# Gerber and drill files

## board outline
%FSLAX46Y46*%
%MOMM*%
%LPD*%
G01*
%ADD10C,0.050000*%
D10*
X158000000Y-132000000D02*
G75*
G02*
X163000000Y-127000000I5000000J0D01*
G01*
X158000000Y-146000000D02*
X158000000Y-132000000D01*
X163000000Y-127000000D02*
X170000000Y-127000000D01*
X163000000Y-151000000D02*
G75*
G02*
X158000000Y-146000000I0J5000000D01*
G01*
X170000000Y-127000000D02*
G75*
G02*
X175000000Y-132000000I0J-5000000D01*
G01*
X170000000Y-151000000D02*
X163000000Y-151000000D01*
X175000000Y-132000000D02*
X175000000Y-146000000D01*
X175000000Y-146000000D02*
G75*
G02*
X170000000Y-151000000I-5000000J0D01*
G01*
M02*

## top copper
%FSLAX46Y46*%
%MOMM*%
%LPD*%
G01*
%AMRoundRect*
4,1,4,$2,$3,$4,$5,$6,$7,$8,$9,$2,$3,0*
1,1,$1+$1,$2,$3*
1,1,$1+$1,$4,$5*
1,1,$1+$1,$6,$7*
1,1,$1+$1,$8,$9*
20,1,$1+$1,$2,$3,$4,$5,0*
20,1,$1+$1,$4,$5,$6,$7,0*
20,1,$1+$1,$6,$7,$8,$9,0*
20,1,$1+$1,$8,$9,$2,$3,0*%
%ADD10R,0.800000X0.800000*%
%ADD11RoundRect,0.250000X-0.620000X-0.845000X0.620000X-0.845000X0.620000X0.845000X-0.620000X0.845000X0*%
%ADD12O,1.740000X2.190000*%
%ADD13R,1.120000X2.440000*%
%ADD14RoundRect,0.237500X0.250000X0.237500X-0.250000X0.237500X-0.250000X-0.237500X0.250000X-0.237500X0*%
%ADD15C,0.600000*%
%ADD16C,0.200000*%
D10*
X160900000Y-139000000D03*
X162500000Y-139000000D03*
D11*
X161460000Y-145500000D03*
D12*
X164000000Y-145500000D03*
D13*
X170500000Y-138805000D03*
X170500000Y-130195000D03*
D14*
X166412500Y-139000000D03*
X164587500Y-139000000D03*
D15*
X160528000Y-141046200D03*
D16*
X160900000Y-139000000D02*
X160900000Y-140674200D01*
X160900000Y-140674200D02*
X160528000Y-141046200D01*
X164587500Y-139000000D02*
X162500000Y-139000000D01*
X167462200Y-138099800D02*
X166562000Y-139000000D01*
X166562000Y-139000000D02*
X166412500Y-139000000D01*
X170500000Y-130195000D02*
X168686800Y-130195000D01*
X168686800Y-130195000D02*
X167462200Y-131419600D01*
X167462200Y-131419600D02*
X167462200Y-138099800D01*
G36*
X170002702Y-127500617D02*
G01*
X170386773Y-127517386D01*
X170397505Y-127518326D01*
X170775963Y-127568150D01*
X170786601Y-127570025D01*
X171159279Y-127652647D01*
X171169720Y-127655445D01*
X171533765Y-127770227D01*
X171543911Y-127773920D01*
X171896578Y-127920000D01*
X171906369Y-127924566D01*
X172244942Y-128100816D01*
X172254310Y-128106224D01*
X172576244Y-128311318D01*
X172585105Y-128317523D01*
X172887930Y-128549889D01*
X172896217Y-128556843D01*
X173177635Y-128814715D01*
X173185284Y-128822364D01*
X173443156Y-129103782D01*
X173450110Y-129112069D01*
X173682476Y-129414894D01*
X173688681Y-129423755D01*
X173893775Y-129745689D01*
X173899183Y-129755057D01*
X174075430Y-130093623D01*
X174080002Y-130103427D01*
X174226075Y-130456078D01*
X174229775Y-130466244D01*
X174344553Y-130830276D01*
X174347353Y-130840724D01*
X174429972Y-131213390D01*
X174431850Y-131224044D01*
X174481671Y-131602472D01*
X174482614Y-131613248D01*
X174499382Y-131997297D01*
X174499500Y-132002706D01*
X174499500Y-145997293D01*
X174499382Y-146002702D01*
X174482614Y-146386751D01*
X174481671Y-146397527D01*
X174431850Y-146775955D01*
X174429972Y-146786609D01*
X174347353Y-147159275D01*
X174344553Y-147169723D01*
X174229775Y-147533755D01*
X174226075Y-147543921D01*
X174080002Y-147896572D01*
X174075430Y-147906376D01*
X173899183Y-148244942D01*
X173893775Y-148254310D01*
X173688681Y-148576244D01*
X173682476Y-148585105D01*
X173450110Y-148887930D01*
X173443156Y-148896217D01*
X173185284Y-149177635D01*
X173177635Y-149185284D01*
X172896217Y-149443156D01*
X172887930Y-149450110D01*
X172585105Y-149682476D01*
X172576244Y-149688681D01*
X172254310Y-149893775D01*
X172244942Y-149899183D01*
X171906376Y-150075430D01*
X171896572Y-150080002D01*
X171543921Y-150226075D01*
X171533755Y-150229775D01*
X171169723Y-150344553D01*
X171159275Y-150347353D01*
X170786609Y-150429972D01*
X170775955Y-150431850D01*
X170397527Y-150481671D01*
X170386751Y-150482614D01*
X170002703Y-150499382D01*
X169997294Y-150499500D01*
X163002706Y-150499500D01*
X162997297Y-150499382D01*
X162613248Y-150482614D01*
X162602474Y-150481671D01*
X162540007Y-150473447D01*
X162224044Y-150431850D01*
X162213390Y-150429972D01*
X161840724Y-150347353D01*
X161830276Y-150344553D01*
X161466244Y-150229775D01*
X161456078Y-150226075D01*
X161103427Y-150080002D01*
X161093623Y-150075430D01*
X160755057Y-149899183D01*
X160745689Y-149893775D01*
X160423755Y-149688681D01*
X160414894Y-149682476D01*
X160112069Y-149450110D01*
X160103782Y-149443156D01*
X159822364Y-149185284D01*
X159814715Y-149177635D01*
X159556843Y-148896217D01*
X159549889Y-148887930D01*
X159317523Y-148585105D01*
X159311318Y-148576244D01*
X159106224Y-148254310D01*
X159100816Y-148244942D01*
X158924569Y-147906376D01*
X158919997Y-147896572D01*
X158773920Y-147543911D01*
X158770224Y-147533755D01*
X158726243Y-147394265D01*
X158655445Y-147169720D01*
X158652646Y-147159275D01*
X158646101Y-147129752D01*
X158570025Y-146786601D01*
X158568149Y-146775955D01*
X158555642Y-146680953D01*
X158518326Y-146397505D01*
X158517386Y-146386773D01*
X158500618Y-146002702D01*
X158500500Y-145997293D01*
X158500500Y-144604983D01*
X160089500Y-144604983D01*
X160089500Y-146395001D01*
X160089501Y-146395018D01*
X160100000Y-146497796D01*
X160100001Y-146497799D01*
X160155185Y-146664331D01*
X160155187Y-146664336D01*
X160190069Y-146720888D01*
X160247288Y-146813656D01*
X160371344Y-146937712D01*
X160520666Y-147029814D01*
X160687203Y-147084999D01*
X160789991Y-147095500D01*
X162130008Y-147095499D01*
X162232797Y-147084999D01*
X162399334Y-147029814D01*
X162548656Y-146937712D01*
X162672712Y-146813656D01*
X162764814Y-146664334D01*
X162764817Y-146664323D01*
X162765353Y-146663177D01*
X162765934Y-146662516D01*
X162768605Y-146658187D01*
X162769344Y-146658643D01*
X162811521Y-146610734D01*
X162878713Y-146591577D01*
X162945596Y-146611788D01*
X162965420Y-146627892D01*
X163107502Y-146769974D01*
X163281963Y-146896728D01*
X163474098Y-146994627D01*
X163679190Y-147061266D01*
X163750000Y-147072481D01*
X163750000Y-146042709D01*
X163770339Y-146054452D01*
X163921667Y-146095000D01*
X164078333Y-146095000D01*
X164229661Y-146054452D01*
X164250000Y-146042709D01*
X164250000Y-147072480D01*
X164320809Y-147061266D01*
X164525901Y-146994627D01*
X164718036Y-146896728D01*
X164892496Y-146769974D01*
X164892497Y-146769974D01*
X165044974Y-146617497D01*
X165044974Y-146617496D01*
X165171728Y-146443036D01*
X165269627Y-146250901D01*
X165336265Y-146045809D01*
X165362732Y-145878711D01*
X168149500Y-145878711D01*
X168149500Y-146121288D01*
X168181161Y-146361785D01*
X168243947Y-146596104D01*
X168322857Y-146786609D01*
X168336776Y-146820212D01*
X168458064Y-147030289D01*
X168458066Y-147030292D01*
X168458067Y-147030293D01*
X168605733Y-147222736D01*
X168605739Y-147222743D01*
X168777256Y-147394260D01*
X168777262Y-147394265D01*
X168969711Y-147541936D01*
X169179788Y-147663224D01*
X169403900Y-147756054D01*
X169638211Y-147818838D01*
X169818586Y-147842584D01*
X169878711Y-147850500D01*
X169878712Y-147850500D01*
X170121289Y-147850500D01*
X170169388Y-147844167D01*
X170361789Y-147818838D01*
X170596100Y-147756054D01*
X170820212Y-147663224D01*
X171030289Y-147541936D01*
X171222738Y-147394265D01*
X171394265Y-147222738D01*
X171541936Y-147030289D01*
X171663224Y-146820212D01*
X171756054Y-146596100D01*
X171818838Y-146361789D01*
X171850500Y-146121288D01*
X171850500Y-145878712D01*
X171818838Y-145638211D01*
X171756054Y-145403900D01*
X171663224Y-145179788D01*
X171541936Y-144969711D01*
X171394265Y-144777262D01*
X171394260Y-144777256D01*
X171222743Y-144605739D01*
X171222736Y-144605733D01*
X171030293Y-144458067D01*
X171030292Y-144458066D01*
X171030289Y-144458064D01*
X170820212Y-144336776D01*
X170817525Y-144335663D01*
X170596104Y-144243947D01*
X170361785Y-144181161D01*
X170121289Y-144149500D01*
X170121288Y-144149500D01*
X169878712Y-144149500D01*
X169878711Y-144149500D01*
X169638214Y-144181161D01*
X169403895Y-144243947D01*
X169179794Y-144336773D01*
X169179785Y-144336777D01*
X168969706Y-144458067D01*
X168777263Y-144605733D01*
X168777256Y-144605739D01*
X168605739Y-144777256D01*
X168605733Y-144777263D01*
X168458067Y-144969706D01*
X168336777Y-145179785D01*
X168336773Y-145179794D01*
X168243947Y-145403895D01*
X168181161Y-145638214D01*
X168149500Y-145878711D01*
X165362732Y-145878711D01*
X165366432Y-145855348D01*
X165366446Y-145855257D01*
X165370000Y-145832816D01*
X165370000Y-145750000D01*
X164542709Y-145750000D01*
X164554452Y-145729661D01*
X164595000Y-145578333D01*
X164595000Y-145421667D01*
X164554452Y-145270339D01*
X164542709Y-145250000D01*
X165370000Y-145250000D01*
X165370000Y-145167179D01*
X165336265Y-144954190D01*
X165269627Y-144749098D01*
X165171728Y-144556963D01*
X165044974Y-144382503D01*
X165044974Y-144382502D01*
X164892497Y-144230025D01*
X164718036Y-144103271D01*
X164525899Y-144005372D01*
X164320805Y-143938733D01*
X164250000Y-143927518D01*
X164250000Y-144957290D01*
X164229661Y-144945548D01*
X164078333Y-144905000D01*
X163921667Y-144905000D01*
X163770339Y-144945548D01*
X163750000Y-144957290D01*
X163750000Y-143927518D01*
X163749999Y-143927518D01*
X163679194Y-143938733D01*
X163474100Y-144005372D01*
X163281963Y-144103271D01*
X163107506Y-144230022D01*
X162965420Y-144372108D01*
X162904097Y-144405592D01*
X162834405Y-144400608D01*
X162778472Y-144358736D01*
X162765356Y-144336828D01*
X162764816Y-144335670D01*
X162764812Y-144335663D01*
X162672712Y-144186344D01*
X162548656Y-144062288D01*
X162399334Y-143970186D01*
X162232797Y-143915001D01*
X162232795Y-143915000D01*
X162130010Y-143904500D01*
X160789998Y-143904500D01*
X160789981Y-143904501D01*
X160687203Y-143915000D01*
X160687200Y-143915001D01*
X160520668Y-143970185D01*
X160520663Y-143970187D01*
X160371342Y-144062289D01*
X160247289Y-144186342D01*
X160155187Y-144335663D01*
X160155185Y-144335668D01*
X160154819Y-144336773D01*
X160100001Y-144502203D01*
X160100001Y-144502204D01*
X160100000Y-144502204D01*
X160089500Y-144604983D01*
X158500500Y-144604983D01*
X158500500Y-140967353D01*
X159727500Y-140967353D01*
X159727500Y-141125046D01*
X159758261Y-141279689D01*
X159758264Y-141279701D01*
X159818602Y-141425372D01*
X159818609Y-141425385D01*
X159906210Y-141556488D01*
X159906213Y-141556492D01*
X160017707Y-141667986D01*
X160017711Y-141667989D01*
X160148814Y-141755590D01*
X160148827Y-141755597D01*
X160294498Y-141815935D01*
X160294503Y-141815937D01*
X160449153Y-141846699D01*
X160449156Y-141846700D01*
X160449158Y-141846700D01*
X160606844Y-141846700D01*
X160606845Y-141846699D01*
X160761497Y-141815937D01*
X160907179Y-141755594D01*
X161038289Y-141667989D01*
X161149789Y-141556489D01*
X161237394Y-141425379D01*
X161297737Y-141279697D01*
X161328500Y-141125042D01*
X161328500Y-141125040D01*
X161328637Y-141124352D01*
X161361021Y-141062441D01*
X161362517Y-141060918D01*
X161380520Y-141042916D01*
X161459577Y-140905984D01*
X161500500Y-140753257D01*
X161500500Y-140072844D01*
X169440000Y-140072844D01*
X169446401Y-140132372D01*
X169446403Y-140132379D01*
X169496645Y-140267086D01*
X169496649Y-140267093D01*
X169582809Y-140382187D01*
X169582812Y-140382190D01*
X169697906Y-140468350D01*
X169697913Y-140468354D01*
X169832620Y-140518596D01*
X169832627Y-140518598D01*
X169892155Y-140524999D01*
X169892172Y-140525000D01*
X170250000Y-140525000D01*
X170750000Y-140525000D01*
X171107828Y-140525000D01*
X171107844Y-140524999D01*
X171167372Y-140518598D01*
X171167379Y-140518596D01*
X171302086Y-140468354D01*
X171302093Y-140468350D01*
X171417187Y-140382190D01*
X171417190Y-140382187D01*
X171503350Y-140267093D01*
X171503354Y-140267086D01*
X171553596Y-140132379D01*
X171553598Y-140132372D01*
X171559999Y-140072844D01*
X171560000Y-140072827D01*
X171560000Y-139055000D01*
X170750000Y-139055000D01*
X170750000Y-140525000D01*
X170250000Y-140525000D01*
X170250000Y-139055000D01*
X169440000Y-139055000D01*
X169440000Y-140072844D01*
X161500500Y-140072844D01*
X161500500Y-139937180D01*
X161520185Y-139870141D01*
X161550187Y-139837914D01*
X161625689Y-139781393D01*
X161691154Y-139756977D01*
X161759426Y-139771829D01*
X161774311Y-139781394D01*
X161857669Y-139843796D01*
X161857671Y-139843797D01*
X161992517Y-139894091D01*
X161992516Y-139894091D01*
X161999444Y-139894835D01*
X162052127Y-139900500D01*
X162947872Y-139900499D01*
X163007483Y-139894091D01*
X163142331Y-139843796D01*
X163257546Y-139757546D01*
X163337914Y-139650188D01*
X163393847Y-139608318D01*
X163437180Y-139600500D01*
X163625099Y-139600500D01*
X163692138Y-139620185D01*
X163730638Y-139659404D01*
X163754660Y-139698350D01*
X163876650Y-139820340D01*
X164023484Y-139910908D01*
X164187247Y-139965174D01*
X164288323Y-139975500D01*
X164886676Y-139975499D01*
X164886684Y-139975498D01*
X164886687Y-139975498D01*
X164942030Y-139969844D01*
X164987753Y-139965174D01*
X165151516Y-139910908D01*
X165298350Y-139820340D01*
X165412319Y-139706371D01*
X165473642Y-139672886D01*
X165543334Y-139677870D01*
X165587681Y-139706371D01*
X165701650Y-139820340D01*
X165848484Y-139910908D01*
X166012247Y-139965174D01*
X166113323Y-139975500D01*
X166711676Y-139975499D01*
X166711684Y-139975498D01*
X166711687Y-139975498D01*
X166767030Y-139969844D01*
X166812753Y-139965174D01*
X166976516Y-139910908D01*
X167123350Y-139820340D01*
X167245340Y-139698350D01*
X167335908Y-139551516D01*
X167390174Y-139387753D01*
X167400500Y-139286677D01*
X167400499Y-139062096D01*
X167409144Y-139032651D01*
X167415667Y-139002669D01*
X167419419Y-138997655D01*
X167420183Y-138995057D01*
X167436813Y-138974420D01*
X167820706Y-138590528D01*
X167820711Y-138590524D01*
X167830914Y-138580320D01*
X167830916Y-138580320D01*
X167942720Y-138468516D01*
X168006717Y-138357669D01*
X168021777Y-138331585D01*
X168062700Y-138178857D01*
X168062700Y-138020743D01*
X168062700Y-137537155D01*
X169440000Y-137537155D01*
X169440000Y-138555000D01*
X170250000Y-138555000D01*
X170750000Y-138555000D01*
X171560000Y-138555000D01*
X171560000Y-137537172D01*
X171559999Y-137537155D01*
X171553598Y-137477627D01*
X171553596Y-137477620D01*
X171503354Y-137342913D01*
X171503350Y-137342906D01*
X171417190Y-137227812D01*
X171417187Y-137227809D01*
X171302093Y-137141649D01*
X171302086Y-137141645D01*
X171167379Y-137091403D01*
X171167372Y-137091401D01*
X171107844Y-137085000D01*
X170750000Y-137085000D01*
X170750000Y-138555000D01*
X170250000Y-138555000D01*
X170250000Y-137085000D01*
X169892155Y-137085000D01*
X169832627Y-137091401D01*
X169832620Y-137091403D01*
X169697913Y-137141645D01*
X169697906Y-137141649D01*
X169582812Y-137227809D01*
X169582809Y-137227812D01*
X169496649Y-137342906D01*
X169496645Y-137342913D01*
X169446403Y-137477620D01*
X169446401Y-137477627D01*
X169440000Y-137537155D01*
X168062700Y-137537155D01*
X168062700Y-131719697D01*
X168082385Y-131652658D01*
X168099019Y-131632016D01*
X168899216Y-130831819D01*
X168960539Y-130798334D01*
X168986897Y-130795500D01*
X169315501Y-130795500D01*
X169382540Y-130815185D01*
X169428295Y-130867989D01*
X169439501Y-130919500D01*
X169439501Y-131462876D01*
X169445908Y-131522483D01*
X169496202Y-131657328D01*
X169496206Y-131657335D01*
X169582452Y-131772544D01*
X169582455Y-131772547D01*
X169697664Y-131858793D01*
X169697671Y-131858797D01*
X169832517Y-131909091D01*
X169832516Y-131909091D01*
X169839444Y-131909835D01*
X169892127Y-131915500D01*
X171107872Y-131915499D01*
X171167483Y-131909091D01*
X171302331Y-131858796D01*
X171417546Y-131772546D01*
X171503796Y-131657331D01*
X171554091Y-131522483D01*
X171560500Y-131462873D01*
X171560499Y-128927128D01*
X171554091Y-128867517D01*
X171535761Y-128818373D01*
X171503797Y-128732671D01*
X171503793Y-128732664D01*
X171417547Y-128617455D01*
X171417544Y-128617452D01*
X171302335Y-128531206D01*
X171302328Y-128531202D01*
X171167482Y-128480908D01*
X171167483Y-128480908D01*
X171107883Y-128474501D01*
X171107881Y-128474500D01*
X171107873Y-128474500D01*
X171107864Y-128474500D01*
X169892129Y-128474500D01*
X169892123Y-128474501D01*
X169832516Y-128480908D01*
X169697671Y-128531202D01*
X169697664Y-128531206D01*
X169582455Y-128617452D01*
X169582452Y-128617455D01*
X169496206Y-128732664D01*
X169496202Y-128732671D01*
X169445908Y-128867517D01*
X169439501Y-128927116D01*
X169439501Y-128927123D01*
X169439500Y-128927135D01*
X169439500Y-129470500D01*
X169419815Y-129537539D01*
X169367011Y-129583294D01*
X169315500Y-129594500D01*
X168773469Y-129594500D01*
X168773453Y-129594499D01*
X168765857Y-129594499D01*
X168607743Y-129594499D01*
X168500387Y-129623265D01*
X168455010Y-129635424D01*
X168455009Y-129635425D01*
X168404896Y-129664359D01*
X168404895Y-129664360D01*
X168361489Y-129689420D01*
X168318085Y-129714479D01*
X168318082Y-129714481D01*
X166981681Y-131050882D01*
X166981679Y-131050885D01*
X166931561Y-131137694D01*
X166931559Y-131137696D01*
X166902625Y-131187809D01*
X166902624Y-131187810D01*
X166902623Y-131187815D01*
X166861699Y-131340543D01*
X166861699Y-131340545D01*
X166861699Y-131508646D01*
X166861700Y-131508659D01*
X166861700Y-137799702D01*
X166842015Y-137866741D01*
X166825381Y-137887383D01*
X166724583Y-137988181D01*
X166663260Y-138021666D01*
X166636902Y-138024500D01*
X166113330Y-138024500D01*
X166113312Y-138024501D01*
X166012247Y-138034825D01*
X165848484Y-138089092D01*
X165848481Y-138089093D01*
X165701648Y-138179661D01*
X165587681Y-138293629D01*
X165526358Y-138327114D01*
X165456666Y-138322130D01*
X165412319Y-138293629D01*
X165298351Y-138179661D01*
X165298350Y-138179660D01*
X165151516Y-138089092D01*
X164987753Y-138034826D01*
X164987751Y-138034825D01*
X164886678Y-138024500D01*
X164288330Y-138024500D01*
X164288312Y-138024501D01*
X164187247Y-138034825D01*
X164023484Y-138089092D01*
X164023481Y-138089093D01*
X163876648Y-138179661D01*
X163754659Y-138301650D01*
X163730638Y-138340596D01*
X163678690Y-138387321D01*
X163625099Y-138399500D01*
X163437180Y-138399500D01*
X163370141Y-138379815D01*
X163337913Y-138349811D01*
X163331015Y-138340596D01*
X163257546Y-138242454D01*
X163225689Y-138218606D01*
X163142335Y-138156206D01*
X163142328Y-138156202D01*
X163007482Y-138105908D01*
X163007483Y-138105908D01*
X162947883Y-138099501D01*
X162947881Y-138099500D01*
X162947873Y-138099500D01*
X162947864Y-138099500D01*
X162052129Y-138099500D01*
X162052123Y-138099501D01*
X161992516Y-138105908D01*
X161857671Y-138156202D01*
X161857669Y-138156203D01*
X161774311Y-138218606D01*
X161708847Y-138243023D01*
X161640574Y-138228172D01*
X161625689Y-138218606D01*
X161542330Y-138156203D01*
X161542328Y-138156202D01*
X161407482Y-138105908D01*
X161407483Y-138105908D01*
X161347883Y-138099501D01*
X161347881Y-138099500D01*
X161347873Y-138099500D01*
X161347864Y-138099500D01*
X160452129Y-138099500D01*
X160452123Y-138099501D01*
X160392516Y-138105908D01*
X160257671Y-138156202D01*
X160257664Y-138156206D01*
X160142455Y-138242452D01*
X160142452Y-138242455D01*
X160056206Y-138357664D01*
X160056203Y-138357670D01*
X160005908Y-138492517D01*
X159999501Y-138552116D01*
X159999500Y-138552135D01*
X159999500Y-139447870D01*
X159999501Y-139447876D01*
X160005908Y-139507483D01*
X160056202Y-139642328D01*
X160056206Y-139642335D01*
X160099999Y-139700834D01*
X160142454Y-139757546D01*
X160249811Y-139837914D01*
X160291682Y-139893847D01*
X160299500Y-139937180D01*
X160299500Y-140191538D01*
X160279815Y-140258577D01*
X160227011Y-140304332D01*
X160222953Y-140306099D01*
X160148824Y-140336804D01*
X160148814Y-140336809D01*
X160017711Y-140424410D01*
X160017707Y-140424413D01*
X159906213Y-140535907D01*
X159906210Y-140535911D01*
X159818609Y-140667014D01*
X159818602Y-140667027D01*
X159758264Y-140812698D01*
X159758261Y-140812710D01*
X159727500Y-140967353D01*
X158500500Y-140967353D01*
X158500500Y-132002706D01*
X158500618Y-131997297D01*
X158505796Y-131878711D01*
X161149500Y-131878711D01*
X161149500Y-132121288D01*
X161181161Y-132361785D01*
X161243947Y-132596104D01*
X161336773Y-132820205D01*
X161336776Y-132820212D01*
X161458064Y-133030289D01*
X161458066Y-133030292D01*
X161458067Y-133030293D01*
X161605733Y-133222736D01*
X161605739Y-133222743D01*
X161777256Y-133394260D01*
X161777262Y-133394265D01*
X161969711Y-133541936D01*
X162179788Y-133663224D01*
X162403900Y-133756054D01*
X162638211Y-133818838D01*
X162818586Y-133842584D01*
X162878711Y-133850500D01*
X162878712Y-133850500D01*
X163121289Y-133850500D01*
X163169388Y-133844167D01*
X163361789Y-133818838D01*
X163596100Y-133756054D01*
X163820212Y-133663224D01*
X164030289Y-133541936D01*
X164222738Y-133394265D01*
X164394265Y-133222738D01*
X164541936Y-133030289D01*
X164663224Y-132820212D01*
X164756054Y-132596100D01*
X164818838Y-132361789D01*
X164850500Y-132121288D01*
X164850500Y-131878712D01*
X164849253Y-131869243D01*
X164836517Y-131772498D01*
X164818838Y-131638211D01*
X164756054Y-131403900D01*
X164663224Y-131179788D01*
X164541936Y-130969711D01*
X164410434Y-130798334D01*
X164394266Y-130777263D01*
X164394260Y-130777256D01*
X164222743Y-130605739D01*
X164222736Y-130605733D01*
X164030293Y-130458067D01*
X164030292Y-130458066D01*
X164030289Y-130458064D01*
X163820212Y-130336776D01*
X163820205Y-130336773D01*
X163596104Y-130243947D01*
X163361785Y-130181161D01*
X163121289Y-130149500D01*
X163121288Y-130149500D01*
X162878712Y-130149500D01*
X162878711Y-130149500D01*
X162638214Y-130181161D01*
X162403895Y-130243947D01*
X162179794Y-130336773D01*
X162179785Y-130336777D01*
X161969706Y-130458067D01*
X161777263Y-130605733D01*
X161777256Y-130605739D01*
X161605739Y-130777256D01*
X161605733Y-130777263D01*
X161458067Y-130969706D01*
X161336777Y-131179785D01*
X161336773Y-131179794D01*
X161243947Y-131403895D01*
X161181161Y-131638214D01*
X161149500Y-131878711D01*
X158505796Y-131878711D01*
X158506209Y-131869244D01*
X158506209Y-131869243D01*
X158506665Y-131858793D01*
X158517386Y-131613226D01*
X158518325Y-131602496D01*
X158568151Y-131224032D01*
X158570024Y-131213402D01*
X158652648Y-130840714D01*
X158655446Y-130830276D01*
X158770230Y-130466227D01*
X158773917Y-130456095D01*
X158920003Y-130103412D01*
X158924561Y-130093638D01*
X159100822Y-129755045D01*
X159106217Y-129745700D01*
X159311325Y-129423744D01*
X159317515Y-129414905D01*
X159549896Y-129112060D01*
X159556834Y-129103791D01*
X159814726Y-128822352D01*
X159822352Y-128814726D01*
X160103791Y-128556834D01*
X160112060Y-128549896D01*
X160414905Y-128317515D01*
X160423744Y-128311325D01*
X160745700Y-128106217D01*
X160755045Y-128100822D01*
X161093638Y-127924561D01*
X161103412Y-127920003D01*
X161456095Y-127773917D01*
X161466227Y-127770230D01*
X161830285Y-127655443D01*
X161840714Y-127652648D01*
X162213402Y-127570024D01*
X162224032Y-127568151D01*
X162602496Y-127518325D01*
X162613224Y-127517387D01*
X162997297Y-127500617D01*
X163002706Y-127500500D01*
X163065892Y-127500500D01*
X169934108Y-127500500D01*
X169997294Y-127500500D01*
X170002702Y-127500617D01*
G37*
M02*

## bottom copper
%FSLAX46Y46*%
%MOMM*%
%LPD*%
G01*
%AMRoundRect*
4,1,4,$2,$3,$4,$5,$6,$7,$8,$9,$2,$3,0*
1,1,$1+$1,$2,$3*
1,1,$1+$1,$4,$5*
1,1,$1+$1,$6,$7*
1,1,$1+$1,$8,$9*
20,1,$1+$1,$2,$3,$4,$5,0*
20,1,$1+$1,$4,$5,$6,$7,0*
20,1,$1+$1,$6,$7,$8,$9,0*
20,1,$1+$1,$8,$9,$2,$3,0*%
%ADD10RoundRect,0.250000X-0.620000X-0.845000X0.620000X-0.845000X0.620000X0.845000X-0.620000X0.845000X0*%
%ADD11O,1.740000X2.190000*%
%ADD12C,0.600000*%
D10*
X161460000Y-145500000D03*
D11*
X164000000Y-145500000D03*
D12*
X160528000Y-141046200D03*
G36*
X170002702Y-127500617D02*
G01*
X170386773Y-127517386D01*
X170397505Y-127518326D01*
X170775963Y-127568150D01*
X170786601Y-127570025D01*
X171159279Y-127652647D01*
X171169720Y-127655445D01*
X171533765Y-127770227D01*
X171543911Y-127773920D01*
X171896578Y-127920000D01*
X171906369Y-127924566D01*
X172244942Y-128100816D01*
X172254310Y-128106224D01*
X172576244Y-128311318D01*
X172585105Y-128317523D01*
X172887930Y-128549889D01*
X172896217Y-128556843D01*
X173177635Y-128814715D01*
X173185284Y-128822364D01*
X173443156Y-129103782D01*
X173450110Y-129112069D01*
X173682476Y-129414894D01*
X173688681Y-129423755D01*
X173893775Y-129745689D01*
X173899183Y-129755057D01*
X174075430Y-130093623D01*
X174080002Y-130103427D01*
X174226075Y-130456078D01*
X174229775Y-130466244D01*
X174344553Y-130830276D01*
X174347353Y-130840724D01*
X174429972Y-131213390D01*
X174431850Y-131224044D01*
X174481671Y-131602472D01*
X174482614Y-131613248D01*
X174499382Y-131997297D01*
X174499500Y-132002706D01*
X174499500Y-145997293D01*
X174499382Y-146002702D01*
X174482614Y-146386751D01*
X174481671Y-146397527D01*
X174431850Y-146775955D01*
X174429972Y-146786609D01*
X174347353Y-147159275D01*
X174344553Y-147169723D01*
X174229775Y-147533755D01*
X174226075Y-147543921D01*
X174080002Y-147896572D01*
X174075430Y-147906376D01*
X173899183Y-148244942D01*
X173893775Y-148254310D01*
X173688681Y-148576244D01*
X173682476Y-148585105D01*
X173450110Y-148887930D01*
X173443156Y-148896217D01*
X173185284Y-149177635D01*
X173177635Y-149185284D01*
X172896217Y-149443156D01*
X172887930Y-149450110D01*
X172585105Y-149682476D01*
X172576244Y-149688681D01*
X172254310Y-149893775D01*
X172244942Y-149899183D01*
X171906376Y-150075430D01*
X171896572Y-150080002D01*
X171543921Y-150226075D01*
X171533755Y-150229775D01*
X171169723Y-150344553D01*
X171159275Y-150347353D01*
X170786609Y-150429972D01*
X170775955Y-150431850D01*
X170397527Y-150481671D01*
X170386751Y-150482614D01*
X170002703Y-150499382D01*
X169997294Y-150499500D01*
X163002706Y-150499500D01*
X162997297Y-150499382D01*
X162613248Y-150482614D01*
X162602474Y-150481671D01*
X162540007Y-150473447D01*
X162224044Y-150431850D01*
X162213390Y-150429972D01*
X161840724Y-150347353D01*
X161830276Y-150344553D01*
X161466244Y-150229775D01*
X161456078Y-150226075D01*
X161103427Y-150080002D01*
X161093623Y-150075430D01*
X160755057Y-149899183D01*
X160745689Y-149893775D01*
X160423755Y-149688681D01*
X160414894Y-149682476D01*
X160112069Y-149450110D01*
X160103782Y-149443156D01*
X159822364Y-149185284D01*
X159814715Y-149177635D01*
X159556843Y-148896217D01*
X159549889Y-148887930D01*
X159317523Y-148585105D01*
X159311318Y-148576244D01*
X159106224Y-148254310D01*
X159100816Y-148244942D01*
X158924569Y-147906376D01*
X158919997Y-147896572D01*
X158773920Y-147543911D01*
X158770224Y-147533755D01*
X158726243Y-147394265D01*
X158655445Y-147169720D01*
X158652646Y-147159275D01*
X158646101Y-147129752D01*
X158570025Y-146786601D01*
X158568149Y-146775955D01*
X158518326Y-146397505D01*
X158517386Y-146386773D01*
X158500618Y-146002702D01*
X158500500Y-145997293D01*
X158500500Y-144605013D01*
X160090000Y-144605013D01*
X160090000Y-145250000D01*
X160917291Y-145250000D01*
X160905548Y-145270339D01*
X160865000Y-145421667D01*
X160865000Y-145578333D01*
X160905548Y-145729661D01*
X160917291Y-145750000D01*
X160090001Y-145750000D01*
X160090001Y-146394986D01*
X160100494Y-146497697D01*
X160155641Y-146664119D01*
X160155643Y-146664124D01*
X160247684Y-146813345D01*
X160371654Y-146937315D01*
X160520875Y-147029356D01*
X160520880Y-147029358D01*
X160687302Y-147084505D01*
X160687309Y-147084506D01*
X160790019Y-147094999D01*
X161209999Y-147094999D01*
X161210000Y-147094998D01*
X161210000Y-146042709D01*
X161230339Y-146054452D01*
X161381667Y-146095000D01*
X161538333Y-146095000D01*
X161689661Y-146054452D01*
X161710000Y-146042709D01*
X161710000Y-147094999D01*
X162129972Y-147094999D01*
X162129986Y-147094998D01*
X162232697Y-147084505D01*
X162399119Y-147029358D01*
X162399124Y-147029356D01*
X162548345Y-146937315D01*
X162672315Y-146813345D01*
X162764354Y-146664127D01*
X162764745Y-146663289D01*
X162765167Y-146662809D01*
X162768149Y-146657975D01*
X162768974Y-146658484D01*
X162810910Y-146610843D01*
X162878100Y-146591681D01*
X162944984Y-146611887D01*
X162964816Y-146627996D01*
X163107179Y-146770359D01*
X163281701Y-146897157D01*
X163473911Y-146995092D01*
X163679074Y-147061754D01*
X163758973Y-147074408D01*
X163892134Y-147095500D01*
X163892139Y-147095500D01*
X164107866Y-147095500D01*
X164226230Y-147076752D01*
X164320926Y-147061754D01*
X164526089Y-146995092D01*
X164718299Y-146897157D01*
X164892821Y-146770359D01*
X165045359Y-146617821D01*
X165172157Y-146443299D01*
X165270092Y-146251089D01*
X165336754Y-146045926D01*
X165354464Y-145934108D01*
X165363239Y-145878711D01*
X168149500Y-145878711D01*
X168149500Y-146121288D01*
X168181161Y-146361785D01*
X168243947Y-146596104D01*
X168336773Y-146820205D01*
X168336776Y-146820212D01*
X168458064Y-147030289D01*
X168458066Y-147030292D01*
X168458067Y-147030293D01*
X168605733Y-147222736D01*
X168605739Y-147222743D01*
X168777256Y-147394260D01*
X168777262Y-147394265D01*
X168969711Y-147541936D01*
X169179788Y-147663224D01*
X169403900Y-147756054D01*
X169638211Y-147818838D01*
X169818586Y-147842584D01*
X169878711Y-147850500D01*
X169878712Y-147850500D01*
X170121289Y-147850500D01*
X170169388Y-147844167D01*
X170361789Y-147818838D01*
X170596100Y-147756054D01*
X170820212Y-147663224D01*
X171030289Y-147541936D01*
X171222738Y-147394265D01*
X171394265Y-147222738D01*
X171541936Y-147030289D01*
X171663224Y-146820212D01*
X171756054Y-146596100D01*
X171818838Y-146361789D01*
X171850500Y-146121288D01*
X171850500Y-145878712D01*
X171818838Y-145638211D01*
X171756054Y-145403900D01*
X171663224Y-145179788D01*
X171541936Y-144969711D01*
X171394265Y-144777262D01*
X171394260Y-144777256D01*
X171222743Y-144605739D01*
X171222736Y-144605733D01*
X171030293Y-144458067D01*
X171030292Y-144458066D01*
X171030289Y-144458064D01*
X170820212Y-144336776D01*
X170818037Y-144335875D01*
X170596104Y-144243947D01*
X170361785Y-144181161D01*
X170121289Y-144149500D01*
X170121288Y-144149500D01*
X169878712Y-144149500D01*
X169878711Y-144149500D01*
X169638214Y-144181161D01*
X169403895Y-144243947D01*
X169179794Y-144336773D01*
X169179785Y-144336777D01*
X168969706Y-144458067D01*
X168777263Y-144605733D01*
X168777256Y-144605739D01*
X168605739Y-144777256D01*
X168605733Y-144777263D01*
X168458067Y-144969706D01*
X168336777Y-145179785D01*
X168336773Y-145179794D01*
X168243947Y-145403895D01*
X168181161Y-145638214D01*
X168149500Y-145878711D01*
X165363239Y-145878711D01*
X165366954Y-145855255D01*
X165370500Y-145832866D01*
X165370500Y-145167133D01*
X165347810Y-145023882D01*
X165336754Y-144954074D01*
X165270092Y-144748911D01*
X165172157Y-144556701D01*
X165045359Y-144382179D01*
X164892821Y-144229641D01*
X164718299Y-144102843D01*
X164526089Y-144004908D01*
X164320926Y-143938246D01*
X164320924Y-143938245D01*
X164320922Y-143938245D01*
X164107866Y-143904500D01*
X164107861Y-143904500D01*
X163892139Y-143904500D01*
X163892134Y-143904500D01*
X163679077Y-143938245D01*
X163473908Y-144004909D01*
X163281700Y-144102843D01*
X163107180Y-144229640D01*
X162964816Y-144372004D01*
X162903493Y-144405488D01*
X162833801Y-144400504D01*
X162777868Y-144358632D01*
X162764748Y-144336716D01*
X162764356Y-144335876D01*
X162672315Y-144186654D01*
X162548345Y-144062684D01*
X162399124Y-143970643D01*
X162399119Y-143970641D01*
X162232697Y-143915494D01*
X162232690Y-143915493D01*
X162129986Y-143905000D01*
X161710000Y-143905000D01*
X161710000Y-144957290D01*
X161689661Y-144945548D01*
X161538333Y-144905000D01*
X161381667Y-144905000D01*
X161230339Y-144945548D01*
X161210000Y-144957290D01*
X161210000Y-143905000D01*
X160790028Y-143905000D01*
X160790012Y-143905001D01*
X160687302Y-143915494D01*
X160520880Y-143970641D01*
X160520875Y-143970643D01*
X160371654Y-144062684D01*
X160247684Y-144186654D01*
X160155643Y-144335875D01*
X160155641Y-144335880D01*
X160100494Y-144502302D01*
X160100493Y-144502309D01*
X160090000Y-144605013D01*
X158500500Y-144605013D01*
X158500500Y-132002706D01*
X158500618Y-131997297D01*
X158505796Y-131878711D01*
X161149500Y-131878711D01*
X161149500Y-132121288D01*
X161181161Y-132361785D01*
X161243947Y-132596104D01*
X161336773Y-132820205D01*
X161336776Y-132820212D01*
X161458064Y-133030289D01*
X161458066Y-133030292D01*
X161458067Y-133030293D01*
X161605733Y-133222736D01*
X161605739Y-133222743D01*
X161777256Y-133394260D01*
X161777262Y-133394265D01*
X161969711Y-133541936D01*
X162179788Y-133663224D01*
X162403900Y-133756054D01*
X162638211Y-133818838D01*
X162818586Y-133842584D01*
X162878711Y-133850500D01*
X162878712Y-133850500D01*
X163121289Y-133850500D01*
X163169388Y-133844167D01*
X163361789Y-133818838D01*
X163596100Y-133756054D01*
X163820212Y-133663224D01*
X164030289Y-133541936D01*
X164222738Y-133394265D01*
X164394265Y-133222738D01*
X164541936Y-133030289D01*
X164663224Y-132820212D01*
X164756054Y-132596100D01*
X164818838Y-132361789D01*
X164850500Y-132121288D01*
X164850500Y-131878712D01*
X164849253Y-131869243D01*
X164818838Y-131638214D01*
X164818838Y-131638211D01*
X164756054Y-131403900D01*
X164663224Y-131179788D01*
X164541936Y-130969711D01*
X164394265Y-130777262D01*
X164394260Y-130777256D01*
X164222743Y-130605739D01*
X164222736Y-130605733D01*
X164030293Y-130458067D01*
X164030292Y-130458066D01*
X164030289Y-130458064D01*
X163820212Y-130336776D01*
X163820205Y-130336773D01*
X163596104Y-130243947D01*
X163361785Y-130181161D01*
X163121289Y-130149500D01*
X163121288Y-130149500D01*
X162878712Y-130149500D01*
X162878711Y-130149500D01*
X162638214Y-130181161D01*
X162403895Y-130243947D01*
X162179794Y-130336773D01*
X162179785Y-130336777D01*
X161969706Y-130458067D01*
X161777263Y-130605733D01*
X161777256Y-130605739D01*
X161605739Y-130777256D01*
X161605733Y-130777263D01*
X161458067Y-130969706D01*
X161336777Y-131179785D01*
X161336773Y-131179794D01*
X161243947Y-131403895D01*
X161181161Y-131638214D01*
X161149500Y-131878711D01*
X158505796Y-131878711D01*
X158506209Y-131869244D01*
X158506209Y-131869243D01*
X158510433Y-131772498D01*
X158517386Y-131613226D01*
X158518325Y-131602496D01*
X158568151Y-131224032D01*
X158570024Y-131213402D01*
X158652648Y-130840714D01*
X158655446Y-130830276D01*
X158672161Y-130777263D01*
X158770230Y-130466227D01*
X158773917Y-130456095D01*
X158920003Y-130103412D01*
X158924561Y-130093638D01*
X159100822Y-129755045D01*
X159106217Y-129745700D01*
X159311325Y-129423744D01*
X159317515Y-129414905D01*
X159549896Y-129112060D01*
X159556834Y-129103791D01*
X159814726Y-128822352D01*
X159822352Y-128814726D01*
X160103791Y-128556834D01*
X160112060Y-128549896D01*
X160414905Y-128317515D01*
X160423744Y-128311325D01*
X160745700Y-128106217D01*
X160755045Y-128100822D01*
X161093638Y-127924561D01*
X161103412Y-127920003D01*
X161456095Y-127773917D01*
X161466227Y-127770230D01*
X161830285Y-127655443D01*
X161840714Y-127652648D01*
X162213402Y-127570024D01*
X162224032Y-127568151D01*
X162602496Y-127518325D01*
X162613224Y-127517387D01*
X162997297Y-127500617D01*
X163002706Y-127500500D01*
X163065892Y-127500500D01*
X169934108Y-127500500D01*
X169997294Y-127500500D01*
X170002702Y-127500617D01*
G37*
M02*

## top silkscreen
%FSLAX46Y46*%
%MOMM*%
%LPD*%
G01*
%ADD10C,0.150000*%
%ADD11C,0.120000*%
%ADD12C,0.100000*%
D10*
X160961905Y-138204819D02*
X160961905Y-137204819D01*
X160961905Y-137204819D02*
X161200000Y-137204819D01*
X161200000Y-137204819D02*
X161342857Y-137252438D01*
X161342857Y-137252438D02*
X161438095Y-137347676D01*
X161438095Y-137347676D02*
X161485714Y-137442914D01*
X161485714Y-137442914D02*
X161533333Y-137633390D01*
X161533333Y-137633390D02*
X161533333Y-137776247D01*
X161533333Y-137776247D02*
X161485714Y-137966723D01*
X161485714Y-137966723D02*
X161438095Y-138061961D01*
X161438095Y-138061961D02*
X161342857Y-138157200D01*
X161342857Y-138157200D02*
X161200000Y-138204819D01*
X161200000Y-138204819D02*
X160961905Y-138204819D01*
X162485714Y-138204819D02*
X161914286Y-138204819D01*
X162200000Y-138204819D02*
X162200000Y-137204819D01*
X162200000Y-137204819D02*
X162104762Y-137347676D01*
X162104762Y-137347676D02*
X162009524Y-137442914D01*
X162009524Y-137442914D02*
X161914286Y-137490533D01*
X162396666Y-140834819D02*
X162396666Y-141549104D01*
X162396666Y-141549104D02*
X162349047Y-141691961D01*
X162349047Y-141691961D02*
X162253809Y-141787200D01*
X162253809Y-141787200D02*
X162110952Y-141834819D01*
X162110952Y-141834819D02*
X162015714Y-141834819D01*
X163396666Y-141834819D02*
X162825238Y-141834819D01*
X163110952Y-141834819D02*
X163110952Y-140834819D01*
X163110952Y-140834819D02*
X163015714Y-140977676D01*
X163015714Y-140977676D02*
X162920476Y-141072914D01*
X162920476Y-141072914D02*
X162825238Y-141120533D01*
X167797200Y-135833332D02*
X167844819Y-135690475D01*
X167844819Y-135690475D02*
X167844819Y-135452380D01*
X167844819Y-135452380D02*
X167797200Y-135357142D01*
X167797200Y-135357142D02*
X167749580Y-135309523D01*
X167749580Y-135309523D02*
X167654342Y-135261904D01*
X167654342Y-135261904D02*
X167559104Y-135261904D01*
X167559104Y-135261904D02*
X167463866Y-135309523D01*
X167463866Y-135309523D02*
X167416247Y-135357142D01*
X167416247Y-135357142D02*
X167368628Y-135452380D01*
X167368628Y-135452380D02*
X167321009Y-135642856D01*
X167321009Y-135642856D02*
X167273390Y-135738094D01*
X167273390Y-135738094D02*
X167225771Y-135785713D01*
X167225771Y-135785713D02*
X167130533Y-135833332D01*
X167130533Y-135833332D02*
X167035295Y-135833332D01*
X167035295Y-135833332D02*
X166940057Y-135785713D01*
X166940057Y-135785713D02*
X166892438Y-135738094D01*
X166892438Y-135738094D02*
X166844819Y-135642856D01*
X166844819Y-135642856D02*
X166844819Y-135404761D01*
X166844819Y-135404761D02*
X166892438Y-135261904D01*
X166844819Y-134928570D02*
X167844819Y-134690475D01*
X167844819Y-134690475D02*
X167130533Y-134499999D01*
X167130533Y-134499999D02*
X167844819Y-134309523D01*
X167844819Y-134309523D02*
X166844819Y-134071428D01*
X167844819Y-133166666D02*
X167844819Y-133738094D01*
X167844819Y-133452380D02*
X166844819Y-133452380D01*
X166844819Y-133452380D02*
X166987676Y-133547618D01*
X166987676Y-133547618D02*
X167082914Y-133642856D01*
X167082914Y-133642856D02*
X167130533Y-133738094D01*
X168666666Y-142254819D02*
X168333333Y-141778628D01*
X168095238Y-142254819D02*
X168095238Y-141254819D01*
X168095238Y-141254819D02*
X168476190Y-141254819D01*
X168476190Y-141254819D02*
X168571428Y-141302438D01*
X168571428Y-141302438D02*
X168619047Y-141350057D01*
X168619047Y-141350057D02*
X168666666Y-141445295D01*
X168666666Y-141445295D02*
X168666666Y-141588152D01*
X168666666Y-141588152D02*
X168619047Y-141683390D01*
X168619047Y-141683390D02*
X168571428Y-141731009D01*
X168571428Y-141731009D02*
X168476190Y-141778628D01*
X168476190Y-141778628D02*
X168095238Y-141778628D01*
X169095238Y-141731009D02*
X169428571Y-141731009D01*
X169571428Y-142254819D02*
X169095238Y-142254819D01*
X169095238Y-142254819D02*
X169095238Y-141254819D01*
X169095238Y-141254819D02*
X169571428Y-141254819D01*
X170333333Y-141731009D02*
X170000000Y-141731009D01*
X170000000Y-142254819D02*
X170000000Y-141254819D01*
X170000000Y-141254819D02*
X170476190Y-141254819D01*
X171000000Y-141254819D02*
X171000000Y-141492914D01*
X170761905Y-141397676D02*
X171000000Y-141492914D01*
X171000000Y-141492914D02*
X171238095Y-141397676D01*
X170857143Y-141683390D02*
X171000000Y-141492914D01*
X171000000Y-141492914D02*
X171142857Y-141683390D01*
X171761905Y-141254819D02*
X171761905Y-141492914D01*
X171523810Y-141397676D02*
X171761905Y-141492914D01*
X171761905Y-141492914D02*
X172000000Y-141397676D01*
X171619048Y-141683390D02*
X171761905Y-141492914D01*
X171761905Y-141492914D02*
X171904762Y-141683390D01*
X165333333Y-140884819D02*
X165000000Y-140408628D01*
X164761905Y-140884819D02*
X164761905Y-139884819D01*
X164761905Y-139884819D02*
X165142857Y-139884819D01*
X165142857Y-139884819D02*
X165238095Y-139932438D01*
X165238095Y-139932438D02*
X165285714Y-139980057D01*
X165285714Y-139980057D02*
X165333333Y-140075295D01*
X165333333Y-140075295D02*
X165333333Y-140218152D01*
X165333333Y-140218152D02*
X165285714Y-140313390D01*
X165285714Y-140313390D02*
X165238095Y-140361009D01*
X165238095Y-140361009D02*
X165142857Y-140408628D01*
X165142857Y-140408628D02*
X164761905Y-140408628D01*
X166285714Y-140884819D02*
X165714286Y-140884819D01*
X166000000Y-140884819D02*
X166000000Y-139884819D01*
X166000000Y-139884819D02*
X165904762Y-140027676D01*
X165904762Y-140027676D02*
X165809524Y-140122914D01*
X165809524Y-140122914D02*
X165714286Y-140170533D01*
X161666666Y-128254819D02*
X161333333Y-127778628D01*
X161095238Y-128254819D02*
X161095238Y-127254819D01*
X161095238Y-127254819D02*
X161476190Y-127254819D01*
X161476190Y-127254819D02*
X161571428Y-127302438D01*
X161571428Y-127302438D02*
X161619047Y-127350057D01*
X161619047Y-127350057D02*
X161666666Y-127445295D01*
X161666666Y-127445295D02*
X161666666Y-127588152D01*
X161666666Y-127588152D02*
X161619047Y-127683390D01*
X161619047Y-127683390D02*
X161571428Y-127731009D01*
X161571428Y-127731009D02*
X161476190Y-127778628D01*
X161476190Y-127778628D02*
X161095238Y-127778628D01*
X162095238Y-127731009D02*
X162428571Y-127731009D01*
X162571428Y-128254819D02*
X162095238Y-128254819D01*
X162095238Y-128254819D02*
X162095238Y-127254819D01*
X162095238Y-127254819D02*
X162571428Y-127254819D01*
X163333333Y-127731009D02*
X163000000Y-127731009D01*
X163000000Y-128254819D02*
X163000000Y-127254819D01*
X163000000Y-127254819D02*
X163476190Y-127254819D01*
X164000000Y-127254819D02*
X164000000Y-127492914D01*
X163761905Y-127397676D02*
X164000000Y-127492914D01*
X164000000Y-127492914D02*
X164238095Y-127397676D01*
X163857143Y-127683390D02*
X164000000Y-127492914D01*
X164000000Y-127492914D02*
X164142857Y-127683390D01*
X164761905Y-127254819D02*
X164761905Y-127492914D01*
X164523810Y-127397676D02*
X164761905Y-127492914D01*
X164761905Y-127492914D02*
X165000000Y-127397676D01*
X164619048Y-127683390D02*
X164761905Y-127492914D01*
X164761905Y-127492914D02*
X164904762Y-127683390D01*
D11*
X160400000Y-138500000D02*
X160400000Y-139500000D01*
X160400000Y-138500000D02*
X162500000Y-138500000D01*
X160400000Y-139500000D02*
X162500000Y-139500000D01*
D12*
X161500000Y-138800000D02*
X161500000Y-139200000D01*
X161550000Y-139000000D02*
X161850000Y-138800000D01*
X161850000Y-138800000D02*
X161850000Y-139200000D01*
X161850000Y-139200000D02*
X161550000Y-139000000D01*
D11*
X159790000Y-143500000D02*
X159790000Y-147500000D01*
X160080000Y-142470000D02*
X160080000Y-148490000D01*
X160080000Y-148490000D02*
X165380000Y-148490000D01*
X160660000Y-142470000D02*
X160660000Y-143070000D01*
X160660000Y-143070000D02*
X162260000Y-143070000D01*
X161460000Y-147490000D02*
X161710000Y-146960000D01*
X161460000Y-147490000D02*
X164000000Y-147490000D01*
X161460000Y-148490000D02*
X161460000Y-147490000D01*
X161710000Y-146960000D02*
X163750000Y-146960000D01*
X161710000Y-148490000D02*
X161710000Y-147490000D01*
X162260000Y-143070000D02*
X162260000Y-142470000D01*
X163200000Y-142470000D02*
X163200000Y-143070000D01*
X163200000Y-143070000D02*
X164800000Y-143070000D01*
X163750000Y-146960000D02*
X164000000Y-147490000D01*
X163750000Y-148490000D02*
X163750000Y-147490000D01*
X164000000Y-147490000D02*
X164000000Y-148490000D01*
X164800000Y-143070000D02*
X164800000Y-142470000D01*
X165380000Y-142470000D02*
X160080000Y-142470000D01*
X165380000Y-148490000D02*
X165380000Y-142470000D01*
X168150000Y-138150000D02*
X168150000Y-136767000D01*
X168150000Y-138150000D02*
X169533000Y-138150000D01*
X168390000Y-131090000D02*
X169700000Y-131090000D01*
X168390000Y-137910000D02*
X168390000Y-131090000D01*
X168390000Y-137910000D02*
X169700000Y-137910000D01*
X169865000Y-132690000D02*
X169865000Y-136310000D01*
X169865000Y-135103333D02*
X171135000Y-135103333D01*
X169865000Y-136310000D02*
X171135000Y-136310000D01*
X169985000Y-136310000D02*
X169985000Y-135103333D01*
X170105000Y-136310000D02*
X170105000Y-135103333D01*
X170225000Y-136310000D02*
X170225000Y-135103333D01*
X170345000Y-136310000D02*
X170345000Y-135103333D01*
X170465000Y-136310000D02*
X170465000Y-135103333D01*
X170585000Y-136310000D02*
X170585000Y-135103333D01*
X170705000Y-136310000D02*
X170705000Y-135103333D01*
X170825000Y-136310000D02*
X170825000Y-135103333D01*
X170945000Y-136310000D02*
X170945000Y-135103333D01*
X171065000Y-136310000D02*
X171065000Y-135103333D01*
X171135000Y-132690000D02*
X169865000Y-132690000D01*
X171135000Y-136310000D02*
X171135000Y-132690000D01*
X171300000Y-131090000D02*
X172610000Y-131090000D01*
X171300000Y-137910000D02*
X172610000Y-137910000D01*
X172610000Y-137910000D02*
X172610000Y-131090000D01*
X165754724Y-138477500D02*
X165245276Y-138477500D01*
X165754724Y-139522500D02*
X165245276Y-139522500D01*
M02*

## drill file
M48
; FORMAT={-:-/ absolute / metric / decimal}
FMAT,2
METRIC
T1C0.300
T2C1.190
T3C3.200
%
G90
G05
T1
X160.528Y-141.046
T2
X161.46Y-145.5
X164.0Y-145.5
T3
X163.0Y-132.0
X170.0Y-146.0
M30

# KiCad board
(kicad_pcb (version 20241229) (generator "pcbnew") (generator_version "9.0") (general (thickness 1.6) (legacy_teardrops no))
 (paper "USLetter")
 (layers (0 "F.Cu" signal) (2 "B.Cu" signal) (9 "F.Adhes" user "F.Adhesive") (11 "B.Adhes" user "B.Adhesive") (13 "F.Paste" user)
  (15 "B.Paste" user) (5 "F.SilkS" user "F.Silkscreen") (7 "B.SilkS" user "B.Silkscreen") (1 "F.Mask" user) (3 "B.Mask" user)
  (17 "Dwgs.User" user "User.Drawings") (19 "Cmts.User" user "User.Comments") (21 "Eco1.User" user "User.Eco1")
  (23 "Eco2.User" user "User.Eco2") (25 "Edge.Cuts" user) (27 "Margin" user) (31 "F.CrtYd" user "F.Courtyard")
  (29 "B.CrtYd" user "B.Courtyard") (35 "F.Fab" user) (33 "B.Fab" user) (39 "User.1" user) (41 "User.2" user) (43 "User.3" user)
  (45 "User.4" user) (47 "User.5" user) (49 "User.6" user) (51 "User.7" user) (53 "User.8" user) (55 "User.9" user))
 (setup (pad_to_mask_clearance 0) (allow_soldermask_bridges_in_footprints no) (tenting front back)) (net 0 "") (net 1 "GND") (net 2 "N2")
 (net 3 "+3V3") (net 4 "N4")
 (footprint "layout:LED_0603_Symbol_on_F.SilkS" (layer "F.Cu") (at 161.7 139)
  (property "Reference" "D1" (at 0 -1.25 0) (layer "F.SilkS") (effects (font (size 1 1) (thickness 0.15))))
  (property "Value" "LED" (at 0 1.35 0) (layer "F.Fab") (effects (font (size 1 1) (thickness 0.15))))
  (fp_line (start -1.3 -0.5) (end -1.3 0.5) (stroke (width 0.12) (type solid)) (layer "F.SilkS"))
  (fp_line (start -1.3 -0.5) (end 0.8 -0.5) (stroke (width 0.12) (type solid)) (layer "F.SilkS"))
  (fp_line (start -1.3 0.5) (end 0.8 0.5) (stroke (width 0.12) (type solid)) (layer "F.SilkS"))
  (fp_line (start -0.2 -0.2) (end -0.2 0.2) (stroke (width 0.1) (type solid)) (layer "F.SilkS"))
  (fp_line (start -0.15 0) (end 0.15 -0.2) (stroke (width 0.1) (type solid)) (layer "F.SilkS"))
  (fp_line (start 0.15 -0.2) (end 0.15 0.2) (stroke (width 0.1) (type solid)) (layer "F.SilkS"))
  (fp_line (start 0.15 0.2) (end -0.15 0) (stroke (width 0.1) (type solid)) (layer "F.SilkS"))
  (pad "1" smd rect (at -0.8 0 180) (size 0.8 0.8) (layers "F.Cu" "F.Mask" "F.Paste") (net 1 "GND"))
  (pad "2" smd rect (at 0.8 0 180) (size 0.8 0.8) (layers "F.Cu" "F.Mask" "F.Paste") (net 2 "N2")))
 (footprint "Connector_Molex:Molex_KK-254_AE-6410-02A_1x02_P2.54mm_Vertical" (layer "F.Cu") (at 161.46 145.5)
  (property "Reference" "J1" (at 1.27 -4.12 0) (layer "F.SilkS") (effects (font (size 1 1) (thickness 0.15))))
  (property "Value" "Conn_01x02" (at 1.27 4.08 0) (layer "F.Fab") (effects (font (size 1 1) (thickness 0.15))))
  (fp_line (start -1.67 -2) (end -1.67 2) (stroke (width 0.12) (type solid)) (layer "F.SilkS"))
  (fp_line (start -1.38 -3.03) (end -1.38 2.99) (stroke (width 0.12) (type solid)) (layer "F.SilkS"))
  (fp_line (start -1.38 2.99) (end 3.92 2.99) (stroke (width 0.12) (type solid)) (layer "F.SilkS"))
  (fp_line (start -0.8 -3.03) (end -0.8 -2.43) (stroke (width 0.12) (type solid)) (layer "F.SilkS"))
  (fp_line (start -0.8 -2.43) (end 0.8 -2.43) (stroke (width 0.12) (type solid)) (layer "F.SilkS"))
  (fp_line (start 0 1.99) (end 0.25 1.46) (stroke (width 0.12) (type solid)) (layer "F.SilkS"))
  (fp_line (start 0 1.99) (end 2.54 1.99) (stroke (width 0.12) (type solid)) (layer "F.SilkS"))
  (fp_line (start 0 2.99) (end 0 1.99) (stroke (width 0.12) (type solid)) (layer "F.SilkS"))
  (fp_line (start 0.25 1.46) (end 2.29 1.46) (stroke (width 0.12) (type solid)) (layer "F.SilkS"))
  (fp_line (start 0.25 2.99) (end 0.25 1.99) (stroke (width 0.12) (type solid)) (layer "F.SilkS"))
  (fp_line (start 0.8 -2.43) (end 0.8 -3.03) (stroke (width 0.12) (type solid)) (layer "F.SilkS"))
  (fp_line (start 1.74 -3.03) (end 1.74 -2.43) (stroke (width 0.12) (type solid)) (layer "F.SilkS"))
  (fp_line (start 1.74 -2.43) (end 3.34 -2.43) (stroke (width 0.12) (type solid)) (layer "F.SilkS"))
  (fp_line (start 2.29 1.46) (end 2.54 1.99) (stroke (width 0.12) (type solid)) (layer "F.SilkS"))
  (fp_line (start 2.29 2.99) (end 2.29 1.99) (stroke (width 0.12) (type solid)) (layer "F.SilkS"))
  (fp_line (start 2.54 1.99) (end 2.54 2.99) (stroke (width 0.12) (type solid)) (layer "F.SilkS"))
  (fp_line (start 3.34 -2.43) (end 3.34 -3.03) (stroke (width 0.12) (type solid)) (layer "F.SilkS"))
  (fp_line (start 3.92 -3.03) (end -1.38 -3.03) (stroke (width 0.12) (type solid)) (layer "F.SilkS"))
  (fp_line (start 3.92 2.99) (end 3.92 -3.03) (stroke (width 0.12) (type solid)) (layer "F.SilkS"))
  (pad "1" thru_hole roundrect (at 0 0) (size 1.74 2.19) (drill 1.19) (layers "*.Cu" "*.Mask") (remove_unused_layers no)
   (roundrect_rratio 0.143678) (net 1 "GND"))
  (pad "2" thru_hole oval (at 2.54 0) (size 1.74 2.19) (drill 1.19) (layers "*.Cu" "*.Mask") (remove_unused_layers no) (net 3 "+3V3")))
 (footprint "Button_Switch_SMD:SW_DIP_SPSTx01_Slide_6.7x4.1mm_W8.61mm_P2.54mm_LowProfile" (layer "F.Cu") (at 170.5 134.5 90)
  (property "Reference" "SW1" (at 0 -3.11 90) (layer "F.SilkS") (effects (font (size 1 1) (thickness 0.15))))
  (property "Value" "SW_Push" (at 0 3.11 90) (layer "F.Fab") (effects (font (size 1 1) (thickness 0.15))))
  (fp_line (start -3.65 -2.35) (end -2.267 -2.35) (stroke (width 0.12) (type solid)) (layer "F.SilkS"))
  (fp_line (start -3.65 -2.35) (end -3.65 -0.967) (stroke (width 0.12) (type solid)) (layer "F.SilkS"))
  (fp_line (start 3.41 -2.11) (end 3.41 -0.8) (stroke (width 0.12) (type solid)) (layer "F.SilkS"))
  (fp_line (start -3.41 -2.11) (end 3.41 -2.11) (stroke (width 0.12) (type solid)) (layer "F.SilkS"))
  (fp_line (start -3.41 -2.11) (end -3.41 -0.8) (stroke (width 0.12) (type solid)) (layer "F.SilkS"))
  (fp_line (start 1.81 -0.635) (end -1.81 -0.635) (stroke (width 0.12) (type solid)) (layer "F.SilkS"))
  (fp_line (start -0.603333 -0.635) (end -0.603333 0.635) (stroke (width 0.12) (type solid)) (layer "F.SilkS"))
  (fp_line (start -1.81 -0.635) (end -1.81 0.635) (stroke (width 0.12) (type solid)) (layer "F.SilkS"))
  (fp_line (start -1.81 -0.515) (end -0.603333 -0.515) (stroke (width 0.12) (type solid)) (layer "F.SilkS"))
  (fp_line (start -1.81 -0.395) (end -0.603333 -0.395) (stroke (width 0.12) (type solid)) (layer "F.SilkS"))
  (fp_line (start -1.81 -0.275) (end -0.603333 -0.275) (stroke (width 0.12) (type solid)) (layer "F.SilkS"))
  (fp_line (start -1.81 -0.155) (end -0.603333 -0.155) (stroke (width 0.12) (type solid)) (layer "F.SilkS"))
  (fp_line (start -1.81 -0.035) (end -0.603333 -0.035) (stroke (width 0.12) (type solid)) (layer "F.SilkS"))
  (fp_line (start -1.81 0.085) (end -0.603333 0.085) (stroke (width 0.12) (type solid)) (layer "F.SilkS"))
  (fp_line (start -1.81 0.205) (end -0.603333 0.205) (stroke (width 0.12) (type solid)) (layer "F.SilkS"))
  (fp_line (start -1.81 0.325) (end -0.603333 0.325) (stroke (width 0.12) (type solid)) (layer "F.SilkS"))
  (fp_line (start -1.81 0.445) (end -0.603333 0.445) (stroke (width 0.12) (type solid)) (layer "F.SilkS"))
  (fp_line (start -1.81 0.565) (end -0.603333 0.565) (stroke (width 0.12) (type solid)) (layer "F.SilkS"))
  (fp_line (start 1.81 0.635) (end 1.81 -0.635) (stroke (width 0.12) (type solid)) (layer "F.SilkS"))
  (fp_line (start -1.81 0.635) (end 1.81 0.635) (stroke (width 0.12) (type solid)) (layer "F.SilkS"))
  (fp_line (start 3.41 0.8) (end 3.41 2.11) (stroke (width 0.12) (type solid)) (layer "F.SilkS"))
  (fp_line (start -3.41 0.8) (end -3.41 2.11) (stroke (width 0.12) (type solid)) (layer "F.SilkS"))
  (fp_line (start -3.41 2.11) (end 3.41 2.11) (stroke (width 0.12) (type solid)) (layer "F.SilkS"))
  (pad "1" smd rect (at -4.305 0 90) (size 2.44 1.12) (layers "F.Cu" "F.Mask" "F.Paste") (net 3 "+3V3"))
  (pad "2" smd rect (at 4.305 0 90) (size 2.44 1.12) (layers "F.Cu" "F.Mask" "F.Paste") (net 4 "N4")))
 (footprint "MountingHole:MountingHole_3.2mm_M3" (layer "F.Cu") (at 170 146)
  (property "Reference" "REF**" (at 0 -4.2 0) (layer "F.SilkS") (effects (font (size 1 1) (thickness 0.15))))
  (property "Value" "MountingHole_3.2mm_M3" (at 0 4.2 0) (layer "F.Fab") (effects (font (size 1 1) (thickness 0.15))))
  (pad "" np_thru_hole circle (at 0 0) (size 3.2 3.2) (drill 3.2) (layers "*.Cu" "*.Mask")))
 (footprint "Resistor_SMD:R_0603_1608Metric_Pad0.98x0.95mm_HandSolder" (layer "F.Cu") (at 165.5 139 180)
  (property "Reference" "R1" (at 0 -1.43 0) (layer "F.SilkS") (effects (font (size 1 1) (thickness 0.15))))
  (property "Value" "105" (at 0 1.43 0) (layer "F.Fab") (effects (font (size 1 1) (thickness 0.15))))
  (fp_line (start -0.254724 0.5225) (end 0.254724 0.5225) (stroke (width 0.12) (type solid)) (layer "F.SilkS"))
  (fp_line (start -0.254724 -0.5225) (end 0.254724 -0.5225) (stroke (width 0.12) (type solid)) (layer "F.SilkS"))
  (pad "1" smd roundrect (at -0.9125 0 180) (size 0.975 0.95) (layers "F.Cu" "F.Mask" "F.Paste") (roundrect_rratio 0.25) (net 4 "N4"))
  (pad "2" smd roundrect (at 0.9125 0 180) (size 0.975 0.95) (layers "F.Cu" "F.Mask" "F.Paste") (roundrect_rratio 0.25) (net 2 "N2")))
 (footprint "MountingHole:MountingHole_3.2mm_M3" (layer "F.Cu") (at 163 132)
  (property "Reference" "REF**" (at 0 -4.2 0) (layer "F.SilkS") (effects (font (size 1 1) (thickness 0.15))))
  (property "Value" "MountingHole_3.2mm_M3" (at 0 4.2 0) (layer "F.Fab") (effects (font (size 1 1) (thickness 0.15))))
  (pad "" np_thru_hole circle (at 0 0) (size 3.2 3.2) (drill 3.2) (layers "*.Cu" "*.Mask")))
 (gr_arc (start 158 132) (mid 159.464466 128.464466) (end 163 127) (stroke (width 0.05) (type default)) (layer "Edge.Cuts"))
 (gr_line (start 158 146) (end 158 132) (stroke (width 0.05) (type default)) (layer "Edge.Cuts"))
 (gr_line (start 163 127) (end 170 127) (stroke (width 0.05) (type default)) (layer "Edge.Cuts"))
 (gr_arc (start 163 151) (mid 159.464466 149.535534) (end 158 146) (stroke (width 0.05) (type default)) (layer "Edge.Cuts"))
 (gr_arc (start 170 127) (mid 173.535534 128.464466) (end 175 132) (stroke (width 0.05) (type default)) (layer "Edge.Cuts"))
 (gr_line (start 170 151) (end 163 151) (stroke (width 0.05) (type default)) (layer "Edge.Cuts"))
 (gr_line (start 175 132) (end 175 146) (stroke (width 0.05) (type default)) (layer "Edge.Cuts"))
 (gr_arc (start 175 146) (mid 173.535534 149.535534) (end 170 151) (stroke (width 0.05) (type default)) (layer "Edge.Cuts"))
 (segment (start 160.9 139) (end 160.9 140.6742) (width 0.2) (layer "F.Cu") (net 1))
 (segment (start 160.9 140.6742) (end 160.528 141.0462) (width 0.2) (layer "F.Cu") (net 1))
 (via (at 160.528 141.0462) (size 0.6) (drill 0.3) (layers "F.Cu" "B.Cu") (free yes) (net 1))
 (segment (start 164.5875 139) (end 162.5 139) (width 0.2) (layer "F.Cu") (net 2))
 (segment (start 167.4622 138.0998) (end 166.562 139) (width 0.2) (layer "F.Cu") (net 4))
 (segment (start 166.562 139) (end 166.4125 139) (width 0.2) (layer "F.Cu") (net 4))
 (segment (start 170.5 130.195) (end 168.6868 130.195) (width 0.2) (layer "F.Cu") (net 4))
 (segment (start 168.6868 130.195) (end 167.4622 131.4196) (width 0.2) (layer "F.Cu") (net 4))
 (segment (start 167.4622 131.4196) (end 167.4622 138.0998) (width 0.2) (layer "F.Cu") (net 4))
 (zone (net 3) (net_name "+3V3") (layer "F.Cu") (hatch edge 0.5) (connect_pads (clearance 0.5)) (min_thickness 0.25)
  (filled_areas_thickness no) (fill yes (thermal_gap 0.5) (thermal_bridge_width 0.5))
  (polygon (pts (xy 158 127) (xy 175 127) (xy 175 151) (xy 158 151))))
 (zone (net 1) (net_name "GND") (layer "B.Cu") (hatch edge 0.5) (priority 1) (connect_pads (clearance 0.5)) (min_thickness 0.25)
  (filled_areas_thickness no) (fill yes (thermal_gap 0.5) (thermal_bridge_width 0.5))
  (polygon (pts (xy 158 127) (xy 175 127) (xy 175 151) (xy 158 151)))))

